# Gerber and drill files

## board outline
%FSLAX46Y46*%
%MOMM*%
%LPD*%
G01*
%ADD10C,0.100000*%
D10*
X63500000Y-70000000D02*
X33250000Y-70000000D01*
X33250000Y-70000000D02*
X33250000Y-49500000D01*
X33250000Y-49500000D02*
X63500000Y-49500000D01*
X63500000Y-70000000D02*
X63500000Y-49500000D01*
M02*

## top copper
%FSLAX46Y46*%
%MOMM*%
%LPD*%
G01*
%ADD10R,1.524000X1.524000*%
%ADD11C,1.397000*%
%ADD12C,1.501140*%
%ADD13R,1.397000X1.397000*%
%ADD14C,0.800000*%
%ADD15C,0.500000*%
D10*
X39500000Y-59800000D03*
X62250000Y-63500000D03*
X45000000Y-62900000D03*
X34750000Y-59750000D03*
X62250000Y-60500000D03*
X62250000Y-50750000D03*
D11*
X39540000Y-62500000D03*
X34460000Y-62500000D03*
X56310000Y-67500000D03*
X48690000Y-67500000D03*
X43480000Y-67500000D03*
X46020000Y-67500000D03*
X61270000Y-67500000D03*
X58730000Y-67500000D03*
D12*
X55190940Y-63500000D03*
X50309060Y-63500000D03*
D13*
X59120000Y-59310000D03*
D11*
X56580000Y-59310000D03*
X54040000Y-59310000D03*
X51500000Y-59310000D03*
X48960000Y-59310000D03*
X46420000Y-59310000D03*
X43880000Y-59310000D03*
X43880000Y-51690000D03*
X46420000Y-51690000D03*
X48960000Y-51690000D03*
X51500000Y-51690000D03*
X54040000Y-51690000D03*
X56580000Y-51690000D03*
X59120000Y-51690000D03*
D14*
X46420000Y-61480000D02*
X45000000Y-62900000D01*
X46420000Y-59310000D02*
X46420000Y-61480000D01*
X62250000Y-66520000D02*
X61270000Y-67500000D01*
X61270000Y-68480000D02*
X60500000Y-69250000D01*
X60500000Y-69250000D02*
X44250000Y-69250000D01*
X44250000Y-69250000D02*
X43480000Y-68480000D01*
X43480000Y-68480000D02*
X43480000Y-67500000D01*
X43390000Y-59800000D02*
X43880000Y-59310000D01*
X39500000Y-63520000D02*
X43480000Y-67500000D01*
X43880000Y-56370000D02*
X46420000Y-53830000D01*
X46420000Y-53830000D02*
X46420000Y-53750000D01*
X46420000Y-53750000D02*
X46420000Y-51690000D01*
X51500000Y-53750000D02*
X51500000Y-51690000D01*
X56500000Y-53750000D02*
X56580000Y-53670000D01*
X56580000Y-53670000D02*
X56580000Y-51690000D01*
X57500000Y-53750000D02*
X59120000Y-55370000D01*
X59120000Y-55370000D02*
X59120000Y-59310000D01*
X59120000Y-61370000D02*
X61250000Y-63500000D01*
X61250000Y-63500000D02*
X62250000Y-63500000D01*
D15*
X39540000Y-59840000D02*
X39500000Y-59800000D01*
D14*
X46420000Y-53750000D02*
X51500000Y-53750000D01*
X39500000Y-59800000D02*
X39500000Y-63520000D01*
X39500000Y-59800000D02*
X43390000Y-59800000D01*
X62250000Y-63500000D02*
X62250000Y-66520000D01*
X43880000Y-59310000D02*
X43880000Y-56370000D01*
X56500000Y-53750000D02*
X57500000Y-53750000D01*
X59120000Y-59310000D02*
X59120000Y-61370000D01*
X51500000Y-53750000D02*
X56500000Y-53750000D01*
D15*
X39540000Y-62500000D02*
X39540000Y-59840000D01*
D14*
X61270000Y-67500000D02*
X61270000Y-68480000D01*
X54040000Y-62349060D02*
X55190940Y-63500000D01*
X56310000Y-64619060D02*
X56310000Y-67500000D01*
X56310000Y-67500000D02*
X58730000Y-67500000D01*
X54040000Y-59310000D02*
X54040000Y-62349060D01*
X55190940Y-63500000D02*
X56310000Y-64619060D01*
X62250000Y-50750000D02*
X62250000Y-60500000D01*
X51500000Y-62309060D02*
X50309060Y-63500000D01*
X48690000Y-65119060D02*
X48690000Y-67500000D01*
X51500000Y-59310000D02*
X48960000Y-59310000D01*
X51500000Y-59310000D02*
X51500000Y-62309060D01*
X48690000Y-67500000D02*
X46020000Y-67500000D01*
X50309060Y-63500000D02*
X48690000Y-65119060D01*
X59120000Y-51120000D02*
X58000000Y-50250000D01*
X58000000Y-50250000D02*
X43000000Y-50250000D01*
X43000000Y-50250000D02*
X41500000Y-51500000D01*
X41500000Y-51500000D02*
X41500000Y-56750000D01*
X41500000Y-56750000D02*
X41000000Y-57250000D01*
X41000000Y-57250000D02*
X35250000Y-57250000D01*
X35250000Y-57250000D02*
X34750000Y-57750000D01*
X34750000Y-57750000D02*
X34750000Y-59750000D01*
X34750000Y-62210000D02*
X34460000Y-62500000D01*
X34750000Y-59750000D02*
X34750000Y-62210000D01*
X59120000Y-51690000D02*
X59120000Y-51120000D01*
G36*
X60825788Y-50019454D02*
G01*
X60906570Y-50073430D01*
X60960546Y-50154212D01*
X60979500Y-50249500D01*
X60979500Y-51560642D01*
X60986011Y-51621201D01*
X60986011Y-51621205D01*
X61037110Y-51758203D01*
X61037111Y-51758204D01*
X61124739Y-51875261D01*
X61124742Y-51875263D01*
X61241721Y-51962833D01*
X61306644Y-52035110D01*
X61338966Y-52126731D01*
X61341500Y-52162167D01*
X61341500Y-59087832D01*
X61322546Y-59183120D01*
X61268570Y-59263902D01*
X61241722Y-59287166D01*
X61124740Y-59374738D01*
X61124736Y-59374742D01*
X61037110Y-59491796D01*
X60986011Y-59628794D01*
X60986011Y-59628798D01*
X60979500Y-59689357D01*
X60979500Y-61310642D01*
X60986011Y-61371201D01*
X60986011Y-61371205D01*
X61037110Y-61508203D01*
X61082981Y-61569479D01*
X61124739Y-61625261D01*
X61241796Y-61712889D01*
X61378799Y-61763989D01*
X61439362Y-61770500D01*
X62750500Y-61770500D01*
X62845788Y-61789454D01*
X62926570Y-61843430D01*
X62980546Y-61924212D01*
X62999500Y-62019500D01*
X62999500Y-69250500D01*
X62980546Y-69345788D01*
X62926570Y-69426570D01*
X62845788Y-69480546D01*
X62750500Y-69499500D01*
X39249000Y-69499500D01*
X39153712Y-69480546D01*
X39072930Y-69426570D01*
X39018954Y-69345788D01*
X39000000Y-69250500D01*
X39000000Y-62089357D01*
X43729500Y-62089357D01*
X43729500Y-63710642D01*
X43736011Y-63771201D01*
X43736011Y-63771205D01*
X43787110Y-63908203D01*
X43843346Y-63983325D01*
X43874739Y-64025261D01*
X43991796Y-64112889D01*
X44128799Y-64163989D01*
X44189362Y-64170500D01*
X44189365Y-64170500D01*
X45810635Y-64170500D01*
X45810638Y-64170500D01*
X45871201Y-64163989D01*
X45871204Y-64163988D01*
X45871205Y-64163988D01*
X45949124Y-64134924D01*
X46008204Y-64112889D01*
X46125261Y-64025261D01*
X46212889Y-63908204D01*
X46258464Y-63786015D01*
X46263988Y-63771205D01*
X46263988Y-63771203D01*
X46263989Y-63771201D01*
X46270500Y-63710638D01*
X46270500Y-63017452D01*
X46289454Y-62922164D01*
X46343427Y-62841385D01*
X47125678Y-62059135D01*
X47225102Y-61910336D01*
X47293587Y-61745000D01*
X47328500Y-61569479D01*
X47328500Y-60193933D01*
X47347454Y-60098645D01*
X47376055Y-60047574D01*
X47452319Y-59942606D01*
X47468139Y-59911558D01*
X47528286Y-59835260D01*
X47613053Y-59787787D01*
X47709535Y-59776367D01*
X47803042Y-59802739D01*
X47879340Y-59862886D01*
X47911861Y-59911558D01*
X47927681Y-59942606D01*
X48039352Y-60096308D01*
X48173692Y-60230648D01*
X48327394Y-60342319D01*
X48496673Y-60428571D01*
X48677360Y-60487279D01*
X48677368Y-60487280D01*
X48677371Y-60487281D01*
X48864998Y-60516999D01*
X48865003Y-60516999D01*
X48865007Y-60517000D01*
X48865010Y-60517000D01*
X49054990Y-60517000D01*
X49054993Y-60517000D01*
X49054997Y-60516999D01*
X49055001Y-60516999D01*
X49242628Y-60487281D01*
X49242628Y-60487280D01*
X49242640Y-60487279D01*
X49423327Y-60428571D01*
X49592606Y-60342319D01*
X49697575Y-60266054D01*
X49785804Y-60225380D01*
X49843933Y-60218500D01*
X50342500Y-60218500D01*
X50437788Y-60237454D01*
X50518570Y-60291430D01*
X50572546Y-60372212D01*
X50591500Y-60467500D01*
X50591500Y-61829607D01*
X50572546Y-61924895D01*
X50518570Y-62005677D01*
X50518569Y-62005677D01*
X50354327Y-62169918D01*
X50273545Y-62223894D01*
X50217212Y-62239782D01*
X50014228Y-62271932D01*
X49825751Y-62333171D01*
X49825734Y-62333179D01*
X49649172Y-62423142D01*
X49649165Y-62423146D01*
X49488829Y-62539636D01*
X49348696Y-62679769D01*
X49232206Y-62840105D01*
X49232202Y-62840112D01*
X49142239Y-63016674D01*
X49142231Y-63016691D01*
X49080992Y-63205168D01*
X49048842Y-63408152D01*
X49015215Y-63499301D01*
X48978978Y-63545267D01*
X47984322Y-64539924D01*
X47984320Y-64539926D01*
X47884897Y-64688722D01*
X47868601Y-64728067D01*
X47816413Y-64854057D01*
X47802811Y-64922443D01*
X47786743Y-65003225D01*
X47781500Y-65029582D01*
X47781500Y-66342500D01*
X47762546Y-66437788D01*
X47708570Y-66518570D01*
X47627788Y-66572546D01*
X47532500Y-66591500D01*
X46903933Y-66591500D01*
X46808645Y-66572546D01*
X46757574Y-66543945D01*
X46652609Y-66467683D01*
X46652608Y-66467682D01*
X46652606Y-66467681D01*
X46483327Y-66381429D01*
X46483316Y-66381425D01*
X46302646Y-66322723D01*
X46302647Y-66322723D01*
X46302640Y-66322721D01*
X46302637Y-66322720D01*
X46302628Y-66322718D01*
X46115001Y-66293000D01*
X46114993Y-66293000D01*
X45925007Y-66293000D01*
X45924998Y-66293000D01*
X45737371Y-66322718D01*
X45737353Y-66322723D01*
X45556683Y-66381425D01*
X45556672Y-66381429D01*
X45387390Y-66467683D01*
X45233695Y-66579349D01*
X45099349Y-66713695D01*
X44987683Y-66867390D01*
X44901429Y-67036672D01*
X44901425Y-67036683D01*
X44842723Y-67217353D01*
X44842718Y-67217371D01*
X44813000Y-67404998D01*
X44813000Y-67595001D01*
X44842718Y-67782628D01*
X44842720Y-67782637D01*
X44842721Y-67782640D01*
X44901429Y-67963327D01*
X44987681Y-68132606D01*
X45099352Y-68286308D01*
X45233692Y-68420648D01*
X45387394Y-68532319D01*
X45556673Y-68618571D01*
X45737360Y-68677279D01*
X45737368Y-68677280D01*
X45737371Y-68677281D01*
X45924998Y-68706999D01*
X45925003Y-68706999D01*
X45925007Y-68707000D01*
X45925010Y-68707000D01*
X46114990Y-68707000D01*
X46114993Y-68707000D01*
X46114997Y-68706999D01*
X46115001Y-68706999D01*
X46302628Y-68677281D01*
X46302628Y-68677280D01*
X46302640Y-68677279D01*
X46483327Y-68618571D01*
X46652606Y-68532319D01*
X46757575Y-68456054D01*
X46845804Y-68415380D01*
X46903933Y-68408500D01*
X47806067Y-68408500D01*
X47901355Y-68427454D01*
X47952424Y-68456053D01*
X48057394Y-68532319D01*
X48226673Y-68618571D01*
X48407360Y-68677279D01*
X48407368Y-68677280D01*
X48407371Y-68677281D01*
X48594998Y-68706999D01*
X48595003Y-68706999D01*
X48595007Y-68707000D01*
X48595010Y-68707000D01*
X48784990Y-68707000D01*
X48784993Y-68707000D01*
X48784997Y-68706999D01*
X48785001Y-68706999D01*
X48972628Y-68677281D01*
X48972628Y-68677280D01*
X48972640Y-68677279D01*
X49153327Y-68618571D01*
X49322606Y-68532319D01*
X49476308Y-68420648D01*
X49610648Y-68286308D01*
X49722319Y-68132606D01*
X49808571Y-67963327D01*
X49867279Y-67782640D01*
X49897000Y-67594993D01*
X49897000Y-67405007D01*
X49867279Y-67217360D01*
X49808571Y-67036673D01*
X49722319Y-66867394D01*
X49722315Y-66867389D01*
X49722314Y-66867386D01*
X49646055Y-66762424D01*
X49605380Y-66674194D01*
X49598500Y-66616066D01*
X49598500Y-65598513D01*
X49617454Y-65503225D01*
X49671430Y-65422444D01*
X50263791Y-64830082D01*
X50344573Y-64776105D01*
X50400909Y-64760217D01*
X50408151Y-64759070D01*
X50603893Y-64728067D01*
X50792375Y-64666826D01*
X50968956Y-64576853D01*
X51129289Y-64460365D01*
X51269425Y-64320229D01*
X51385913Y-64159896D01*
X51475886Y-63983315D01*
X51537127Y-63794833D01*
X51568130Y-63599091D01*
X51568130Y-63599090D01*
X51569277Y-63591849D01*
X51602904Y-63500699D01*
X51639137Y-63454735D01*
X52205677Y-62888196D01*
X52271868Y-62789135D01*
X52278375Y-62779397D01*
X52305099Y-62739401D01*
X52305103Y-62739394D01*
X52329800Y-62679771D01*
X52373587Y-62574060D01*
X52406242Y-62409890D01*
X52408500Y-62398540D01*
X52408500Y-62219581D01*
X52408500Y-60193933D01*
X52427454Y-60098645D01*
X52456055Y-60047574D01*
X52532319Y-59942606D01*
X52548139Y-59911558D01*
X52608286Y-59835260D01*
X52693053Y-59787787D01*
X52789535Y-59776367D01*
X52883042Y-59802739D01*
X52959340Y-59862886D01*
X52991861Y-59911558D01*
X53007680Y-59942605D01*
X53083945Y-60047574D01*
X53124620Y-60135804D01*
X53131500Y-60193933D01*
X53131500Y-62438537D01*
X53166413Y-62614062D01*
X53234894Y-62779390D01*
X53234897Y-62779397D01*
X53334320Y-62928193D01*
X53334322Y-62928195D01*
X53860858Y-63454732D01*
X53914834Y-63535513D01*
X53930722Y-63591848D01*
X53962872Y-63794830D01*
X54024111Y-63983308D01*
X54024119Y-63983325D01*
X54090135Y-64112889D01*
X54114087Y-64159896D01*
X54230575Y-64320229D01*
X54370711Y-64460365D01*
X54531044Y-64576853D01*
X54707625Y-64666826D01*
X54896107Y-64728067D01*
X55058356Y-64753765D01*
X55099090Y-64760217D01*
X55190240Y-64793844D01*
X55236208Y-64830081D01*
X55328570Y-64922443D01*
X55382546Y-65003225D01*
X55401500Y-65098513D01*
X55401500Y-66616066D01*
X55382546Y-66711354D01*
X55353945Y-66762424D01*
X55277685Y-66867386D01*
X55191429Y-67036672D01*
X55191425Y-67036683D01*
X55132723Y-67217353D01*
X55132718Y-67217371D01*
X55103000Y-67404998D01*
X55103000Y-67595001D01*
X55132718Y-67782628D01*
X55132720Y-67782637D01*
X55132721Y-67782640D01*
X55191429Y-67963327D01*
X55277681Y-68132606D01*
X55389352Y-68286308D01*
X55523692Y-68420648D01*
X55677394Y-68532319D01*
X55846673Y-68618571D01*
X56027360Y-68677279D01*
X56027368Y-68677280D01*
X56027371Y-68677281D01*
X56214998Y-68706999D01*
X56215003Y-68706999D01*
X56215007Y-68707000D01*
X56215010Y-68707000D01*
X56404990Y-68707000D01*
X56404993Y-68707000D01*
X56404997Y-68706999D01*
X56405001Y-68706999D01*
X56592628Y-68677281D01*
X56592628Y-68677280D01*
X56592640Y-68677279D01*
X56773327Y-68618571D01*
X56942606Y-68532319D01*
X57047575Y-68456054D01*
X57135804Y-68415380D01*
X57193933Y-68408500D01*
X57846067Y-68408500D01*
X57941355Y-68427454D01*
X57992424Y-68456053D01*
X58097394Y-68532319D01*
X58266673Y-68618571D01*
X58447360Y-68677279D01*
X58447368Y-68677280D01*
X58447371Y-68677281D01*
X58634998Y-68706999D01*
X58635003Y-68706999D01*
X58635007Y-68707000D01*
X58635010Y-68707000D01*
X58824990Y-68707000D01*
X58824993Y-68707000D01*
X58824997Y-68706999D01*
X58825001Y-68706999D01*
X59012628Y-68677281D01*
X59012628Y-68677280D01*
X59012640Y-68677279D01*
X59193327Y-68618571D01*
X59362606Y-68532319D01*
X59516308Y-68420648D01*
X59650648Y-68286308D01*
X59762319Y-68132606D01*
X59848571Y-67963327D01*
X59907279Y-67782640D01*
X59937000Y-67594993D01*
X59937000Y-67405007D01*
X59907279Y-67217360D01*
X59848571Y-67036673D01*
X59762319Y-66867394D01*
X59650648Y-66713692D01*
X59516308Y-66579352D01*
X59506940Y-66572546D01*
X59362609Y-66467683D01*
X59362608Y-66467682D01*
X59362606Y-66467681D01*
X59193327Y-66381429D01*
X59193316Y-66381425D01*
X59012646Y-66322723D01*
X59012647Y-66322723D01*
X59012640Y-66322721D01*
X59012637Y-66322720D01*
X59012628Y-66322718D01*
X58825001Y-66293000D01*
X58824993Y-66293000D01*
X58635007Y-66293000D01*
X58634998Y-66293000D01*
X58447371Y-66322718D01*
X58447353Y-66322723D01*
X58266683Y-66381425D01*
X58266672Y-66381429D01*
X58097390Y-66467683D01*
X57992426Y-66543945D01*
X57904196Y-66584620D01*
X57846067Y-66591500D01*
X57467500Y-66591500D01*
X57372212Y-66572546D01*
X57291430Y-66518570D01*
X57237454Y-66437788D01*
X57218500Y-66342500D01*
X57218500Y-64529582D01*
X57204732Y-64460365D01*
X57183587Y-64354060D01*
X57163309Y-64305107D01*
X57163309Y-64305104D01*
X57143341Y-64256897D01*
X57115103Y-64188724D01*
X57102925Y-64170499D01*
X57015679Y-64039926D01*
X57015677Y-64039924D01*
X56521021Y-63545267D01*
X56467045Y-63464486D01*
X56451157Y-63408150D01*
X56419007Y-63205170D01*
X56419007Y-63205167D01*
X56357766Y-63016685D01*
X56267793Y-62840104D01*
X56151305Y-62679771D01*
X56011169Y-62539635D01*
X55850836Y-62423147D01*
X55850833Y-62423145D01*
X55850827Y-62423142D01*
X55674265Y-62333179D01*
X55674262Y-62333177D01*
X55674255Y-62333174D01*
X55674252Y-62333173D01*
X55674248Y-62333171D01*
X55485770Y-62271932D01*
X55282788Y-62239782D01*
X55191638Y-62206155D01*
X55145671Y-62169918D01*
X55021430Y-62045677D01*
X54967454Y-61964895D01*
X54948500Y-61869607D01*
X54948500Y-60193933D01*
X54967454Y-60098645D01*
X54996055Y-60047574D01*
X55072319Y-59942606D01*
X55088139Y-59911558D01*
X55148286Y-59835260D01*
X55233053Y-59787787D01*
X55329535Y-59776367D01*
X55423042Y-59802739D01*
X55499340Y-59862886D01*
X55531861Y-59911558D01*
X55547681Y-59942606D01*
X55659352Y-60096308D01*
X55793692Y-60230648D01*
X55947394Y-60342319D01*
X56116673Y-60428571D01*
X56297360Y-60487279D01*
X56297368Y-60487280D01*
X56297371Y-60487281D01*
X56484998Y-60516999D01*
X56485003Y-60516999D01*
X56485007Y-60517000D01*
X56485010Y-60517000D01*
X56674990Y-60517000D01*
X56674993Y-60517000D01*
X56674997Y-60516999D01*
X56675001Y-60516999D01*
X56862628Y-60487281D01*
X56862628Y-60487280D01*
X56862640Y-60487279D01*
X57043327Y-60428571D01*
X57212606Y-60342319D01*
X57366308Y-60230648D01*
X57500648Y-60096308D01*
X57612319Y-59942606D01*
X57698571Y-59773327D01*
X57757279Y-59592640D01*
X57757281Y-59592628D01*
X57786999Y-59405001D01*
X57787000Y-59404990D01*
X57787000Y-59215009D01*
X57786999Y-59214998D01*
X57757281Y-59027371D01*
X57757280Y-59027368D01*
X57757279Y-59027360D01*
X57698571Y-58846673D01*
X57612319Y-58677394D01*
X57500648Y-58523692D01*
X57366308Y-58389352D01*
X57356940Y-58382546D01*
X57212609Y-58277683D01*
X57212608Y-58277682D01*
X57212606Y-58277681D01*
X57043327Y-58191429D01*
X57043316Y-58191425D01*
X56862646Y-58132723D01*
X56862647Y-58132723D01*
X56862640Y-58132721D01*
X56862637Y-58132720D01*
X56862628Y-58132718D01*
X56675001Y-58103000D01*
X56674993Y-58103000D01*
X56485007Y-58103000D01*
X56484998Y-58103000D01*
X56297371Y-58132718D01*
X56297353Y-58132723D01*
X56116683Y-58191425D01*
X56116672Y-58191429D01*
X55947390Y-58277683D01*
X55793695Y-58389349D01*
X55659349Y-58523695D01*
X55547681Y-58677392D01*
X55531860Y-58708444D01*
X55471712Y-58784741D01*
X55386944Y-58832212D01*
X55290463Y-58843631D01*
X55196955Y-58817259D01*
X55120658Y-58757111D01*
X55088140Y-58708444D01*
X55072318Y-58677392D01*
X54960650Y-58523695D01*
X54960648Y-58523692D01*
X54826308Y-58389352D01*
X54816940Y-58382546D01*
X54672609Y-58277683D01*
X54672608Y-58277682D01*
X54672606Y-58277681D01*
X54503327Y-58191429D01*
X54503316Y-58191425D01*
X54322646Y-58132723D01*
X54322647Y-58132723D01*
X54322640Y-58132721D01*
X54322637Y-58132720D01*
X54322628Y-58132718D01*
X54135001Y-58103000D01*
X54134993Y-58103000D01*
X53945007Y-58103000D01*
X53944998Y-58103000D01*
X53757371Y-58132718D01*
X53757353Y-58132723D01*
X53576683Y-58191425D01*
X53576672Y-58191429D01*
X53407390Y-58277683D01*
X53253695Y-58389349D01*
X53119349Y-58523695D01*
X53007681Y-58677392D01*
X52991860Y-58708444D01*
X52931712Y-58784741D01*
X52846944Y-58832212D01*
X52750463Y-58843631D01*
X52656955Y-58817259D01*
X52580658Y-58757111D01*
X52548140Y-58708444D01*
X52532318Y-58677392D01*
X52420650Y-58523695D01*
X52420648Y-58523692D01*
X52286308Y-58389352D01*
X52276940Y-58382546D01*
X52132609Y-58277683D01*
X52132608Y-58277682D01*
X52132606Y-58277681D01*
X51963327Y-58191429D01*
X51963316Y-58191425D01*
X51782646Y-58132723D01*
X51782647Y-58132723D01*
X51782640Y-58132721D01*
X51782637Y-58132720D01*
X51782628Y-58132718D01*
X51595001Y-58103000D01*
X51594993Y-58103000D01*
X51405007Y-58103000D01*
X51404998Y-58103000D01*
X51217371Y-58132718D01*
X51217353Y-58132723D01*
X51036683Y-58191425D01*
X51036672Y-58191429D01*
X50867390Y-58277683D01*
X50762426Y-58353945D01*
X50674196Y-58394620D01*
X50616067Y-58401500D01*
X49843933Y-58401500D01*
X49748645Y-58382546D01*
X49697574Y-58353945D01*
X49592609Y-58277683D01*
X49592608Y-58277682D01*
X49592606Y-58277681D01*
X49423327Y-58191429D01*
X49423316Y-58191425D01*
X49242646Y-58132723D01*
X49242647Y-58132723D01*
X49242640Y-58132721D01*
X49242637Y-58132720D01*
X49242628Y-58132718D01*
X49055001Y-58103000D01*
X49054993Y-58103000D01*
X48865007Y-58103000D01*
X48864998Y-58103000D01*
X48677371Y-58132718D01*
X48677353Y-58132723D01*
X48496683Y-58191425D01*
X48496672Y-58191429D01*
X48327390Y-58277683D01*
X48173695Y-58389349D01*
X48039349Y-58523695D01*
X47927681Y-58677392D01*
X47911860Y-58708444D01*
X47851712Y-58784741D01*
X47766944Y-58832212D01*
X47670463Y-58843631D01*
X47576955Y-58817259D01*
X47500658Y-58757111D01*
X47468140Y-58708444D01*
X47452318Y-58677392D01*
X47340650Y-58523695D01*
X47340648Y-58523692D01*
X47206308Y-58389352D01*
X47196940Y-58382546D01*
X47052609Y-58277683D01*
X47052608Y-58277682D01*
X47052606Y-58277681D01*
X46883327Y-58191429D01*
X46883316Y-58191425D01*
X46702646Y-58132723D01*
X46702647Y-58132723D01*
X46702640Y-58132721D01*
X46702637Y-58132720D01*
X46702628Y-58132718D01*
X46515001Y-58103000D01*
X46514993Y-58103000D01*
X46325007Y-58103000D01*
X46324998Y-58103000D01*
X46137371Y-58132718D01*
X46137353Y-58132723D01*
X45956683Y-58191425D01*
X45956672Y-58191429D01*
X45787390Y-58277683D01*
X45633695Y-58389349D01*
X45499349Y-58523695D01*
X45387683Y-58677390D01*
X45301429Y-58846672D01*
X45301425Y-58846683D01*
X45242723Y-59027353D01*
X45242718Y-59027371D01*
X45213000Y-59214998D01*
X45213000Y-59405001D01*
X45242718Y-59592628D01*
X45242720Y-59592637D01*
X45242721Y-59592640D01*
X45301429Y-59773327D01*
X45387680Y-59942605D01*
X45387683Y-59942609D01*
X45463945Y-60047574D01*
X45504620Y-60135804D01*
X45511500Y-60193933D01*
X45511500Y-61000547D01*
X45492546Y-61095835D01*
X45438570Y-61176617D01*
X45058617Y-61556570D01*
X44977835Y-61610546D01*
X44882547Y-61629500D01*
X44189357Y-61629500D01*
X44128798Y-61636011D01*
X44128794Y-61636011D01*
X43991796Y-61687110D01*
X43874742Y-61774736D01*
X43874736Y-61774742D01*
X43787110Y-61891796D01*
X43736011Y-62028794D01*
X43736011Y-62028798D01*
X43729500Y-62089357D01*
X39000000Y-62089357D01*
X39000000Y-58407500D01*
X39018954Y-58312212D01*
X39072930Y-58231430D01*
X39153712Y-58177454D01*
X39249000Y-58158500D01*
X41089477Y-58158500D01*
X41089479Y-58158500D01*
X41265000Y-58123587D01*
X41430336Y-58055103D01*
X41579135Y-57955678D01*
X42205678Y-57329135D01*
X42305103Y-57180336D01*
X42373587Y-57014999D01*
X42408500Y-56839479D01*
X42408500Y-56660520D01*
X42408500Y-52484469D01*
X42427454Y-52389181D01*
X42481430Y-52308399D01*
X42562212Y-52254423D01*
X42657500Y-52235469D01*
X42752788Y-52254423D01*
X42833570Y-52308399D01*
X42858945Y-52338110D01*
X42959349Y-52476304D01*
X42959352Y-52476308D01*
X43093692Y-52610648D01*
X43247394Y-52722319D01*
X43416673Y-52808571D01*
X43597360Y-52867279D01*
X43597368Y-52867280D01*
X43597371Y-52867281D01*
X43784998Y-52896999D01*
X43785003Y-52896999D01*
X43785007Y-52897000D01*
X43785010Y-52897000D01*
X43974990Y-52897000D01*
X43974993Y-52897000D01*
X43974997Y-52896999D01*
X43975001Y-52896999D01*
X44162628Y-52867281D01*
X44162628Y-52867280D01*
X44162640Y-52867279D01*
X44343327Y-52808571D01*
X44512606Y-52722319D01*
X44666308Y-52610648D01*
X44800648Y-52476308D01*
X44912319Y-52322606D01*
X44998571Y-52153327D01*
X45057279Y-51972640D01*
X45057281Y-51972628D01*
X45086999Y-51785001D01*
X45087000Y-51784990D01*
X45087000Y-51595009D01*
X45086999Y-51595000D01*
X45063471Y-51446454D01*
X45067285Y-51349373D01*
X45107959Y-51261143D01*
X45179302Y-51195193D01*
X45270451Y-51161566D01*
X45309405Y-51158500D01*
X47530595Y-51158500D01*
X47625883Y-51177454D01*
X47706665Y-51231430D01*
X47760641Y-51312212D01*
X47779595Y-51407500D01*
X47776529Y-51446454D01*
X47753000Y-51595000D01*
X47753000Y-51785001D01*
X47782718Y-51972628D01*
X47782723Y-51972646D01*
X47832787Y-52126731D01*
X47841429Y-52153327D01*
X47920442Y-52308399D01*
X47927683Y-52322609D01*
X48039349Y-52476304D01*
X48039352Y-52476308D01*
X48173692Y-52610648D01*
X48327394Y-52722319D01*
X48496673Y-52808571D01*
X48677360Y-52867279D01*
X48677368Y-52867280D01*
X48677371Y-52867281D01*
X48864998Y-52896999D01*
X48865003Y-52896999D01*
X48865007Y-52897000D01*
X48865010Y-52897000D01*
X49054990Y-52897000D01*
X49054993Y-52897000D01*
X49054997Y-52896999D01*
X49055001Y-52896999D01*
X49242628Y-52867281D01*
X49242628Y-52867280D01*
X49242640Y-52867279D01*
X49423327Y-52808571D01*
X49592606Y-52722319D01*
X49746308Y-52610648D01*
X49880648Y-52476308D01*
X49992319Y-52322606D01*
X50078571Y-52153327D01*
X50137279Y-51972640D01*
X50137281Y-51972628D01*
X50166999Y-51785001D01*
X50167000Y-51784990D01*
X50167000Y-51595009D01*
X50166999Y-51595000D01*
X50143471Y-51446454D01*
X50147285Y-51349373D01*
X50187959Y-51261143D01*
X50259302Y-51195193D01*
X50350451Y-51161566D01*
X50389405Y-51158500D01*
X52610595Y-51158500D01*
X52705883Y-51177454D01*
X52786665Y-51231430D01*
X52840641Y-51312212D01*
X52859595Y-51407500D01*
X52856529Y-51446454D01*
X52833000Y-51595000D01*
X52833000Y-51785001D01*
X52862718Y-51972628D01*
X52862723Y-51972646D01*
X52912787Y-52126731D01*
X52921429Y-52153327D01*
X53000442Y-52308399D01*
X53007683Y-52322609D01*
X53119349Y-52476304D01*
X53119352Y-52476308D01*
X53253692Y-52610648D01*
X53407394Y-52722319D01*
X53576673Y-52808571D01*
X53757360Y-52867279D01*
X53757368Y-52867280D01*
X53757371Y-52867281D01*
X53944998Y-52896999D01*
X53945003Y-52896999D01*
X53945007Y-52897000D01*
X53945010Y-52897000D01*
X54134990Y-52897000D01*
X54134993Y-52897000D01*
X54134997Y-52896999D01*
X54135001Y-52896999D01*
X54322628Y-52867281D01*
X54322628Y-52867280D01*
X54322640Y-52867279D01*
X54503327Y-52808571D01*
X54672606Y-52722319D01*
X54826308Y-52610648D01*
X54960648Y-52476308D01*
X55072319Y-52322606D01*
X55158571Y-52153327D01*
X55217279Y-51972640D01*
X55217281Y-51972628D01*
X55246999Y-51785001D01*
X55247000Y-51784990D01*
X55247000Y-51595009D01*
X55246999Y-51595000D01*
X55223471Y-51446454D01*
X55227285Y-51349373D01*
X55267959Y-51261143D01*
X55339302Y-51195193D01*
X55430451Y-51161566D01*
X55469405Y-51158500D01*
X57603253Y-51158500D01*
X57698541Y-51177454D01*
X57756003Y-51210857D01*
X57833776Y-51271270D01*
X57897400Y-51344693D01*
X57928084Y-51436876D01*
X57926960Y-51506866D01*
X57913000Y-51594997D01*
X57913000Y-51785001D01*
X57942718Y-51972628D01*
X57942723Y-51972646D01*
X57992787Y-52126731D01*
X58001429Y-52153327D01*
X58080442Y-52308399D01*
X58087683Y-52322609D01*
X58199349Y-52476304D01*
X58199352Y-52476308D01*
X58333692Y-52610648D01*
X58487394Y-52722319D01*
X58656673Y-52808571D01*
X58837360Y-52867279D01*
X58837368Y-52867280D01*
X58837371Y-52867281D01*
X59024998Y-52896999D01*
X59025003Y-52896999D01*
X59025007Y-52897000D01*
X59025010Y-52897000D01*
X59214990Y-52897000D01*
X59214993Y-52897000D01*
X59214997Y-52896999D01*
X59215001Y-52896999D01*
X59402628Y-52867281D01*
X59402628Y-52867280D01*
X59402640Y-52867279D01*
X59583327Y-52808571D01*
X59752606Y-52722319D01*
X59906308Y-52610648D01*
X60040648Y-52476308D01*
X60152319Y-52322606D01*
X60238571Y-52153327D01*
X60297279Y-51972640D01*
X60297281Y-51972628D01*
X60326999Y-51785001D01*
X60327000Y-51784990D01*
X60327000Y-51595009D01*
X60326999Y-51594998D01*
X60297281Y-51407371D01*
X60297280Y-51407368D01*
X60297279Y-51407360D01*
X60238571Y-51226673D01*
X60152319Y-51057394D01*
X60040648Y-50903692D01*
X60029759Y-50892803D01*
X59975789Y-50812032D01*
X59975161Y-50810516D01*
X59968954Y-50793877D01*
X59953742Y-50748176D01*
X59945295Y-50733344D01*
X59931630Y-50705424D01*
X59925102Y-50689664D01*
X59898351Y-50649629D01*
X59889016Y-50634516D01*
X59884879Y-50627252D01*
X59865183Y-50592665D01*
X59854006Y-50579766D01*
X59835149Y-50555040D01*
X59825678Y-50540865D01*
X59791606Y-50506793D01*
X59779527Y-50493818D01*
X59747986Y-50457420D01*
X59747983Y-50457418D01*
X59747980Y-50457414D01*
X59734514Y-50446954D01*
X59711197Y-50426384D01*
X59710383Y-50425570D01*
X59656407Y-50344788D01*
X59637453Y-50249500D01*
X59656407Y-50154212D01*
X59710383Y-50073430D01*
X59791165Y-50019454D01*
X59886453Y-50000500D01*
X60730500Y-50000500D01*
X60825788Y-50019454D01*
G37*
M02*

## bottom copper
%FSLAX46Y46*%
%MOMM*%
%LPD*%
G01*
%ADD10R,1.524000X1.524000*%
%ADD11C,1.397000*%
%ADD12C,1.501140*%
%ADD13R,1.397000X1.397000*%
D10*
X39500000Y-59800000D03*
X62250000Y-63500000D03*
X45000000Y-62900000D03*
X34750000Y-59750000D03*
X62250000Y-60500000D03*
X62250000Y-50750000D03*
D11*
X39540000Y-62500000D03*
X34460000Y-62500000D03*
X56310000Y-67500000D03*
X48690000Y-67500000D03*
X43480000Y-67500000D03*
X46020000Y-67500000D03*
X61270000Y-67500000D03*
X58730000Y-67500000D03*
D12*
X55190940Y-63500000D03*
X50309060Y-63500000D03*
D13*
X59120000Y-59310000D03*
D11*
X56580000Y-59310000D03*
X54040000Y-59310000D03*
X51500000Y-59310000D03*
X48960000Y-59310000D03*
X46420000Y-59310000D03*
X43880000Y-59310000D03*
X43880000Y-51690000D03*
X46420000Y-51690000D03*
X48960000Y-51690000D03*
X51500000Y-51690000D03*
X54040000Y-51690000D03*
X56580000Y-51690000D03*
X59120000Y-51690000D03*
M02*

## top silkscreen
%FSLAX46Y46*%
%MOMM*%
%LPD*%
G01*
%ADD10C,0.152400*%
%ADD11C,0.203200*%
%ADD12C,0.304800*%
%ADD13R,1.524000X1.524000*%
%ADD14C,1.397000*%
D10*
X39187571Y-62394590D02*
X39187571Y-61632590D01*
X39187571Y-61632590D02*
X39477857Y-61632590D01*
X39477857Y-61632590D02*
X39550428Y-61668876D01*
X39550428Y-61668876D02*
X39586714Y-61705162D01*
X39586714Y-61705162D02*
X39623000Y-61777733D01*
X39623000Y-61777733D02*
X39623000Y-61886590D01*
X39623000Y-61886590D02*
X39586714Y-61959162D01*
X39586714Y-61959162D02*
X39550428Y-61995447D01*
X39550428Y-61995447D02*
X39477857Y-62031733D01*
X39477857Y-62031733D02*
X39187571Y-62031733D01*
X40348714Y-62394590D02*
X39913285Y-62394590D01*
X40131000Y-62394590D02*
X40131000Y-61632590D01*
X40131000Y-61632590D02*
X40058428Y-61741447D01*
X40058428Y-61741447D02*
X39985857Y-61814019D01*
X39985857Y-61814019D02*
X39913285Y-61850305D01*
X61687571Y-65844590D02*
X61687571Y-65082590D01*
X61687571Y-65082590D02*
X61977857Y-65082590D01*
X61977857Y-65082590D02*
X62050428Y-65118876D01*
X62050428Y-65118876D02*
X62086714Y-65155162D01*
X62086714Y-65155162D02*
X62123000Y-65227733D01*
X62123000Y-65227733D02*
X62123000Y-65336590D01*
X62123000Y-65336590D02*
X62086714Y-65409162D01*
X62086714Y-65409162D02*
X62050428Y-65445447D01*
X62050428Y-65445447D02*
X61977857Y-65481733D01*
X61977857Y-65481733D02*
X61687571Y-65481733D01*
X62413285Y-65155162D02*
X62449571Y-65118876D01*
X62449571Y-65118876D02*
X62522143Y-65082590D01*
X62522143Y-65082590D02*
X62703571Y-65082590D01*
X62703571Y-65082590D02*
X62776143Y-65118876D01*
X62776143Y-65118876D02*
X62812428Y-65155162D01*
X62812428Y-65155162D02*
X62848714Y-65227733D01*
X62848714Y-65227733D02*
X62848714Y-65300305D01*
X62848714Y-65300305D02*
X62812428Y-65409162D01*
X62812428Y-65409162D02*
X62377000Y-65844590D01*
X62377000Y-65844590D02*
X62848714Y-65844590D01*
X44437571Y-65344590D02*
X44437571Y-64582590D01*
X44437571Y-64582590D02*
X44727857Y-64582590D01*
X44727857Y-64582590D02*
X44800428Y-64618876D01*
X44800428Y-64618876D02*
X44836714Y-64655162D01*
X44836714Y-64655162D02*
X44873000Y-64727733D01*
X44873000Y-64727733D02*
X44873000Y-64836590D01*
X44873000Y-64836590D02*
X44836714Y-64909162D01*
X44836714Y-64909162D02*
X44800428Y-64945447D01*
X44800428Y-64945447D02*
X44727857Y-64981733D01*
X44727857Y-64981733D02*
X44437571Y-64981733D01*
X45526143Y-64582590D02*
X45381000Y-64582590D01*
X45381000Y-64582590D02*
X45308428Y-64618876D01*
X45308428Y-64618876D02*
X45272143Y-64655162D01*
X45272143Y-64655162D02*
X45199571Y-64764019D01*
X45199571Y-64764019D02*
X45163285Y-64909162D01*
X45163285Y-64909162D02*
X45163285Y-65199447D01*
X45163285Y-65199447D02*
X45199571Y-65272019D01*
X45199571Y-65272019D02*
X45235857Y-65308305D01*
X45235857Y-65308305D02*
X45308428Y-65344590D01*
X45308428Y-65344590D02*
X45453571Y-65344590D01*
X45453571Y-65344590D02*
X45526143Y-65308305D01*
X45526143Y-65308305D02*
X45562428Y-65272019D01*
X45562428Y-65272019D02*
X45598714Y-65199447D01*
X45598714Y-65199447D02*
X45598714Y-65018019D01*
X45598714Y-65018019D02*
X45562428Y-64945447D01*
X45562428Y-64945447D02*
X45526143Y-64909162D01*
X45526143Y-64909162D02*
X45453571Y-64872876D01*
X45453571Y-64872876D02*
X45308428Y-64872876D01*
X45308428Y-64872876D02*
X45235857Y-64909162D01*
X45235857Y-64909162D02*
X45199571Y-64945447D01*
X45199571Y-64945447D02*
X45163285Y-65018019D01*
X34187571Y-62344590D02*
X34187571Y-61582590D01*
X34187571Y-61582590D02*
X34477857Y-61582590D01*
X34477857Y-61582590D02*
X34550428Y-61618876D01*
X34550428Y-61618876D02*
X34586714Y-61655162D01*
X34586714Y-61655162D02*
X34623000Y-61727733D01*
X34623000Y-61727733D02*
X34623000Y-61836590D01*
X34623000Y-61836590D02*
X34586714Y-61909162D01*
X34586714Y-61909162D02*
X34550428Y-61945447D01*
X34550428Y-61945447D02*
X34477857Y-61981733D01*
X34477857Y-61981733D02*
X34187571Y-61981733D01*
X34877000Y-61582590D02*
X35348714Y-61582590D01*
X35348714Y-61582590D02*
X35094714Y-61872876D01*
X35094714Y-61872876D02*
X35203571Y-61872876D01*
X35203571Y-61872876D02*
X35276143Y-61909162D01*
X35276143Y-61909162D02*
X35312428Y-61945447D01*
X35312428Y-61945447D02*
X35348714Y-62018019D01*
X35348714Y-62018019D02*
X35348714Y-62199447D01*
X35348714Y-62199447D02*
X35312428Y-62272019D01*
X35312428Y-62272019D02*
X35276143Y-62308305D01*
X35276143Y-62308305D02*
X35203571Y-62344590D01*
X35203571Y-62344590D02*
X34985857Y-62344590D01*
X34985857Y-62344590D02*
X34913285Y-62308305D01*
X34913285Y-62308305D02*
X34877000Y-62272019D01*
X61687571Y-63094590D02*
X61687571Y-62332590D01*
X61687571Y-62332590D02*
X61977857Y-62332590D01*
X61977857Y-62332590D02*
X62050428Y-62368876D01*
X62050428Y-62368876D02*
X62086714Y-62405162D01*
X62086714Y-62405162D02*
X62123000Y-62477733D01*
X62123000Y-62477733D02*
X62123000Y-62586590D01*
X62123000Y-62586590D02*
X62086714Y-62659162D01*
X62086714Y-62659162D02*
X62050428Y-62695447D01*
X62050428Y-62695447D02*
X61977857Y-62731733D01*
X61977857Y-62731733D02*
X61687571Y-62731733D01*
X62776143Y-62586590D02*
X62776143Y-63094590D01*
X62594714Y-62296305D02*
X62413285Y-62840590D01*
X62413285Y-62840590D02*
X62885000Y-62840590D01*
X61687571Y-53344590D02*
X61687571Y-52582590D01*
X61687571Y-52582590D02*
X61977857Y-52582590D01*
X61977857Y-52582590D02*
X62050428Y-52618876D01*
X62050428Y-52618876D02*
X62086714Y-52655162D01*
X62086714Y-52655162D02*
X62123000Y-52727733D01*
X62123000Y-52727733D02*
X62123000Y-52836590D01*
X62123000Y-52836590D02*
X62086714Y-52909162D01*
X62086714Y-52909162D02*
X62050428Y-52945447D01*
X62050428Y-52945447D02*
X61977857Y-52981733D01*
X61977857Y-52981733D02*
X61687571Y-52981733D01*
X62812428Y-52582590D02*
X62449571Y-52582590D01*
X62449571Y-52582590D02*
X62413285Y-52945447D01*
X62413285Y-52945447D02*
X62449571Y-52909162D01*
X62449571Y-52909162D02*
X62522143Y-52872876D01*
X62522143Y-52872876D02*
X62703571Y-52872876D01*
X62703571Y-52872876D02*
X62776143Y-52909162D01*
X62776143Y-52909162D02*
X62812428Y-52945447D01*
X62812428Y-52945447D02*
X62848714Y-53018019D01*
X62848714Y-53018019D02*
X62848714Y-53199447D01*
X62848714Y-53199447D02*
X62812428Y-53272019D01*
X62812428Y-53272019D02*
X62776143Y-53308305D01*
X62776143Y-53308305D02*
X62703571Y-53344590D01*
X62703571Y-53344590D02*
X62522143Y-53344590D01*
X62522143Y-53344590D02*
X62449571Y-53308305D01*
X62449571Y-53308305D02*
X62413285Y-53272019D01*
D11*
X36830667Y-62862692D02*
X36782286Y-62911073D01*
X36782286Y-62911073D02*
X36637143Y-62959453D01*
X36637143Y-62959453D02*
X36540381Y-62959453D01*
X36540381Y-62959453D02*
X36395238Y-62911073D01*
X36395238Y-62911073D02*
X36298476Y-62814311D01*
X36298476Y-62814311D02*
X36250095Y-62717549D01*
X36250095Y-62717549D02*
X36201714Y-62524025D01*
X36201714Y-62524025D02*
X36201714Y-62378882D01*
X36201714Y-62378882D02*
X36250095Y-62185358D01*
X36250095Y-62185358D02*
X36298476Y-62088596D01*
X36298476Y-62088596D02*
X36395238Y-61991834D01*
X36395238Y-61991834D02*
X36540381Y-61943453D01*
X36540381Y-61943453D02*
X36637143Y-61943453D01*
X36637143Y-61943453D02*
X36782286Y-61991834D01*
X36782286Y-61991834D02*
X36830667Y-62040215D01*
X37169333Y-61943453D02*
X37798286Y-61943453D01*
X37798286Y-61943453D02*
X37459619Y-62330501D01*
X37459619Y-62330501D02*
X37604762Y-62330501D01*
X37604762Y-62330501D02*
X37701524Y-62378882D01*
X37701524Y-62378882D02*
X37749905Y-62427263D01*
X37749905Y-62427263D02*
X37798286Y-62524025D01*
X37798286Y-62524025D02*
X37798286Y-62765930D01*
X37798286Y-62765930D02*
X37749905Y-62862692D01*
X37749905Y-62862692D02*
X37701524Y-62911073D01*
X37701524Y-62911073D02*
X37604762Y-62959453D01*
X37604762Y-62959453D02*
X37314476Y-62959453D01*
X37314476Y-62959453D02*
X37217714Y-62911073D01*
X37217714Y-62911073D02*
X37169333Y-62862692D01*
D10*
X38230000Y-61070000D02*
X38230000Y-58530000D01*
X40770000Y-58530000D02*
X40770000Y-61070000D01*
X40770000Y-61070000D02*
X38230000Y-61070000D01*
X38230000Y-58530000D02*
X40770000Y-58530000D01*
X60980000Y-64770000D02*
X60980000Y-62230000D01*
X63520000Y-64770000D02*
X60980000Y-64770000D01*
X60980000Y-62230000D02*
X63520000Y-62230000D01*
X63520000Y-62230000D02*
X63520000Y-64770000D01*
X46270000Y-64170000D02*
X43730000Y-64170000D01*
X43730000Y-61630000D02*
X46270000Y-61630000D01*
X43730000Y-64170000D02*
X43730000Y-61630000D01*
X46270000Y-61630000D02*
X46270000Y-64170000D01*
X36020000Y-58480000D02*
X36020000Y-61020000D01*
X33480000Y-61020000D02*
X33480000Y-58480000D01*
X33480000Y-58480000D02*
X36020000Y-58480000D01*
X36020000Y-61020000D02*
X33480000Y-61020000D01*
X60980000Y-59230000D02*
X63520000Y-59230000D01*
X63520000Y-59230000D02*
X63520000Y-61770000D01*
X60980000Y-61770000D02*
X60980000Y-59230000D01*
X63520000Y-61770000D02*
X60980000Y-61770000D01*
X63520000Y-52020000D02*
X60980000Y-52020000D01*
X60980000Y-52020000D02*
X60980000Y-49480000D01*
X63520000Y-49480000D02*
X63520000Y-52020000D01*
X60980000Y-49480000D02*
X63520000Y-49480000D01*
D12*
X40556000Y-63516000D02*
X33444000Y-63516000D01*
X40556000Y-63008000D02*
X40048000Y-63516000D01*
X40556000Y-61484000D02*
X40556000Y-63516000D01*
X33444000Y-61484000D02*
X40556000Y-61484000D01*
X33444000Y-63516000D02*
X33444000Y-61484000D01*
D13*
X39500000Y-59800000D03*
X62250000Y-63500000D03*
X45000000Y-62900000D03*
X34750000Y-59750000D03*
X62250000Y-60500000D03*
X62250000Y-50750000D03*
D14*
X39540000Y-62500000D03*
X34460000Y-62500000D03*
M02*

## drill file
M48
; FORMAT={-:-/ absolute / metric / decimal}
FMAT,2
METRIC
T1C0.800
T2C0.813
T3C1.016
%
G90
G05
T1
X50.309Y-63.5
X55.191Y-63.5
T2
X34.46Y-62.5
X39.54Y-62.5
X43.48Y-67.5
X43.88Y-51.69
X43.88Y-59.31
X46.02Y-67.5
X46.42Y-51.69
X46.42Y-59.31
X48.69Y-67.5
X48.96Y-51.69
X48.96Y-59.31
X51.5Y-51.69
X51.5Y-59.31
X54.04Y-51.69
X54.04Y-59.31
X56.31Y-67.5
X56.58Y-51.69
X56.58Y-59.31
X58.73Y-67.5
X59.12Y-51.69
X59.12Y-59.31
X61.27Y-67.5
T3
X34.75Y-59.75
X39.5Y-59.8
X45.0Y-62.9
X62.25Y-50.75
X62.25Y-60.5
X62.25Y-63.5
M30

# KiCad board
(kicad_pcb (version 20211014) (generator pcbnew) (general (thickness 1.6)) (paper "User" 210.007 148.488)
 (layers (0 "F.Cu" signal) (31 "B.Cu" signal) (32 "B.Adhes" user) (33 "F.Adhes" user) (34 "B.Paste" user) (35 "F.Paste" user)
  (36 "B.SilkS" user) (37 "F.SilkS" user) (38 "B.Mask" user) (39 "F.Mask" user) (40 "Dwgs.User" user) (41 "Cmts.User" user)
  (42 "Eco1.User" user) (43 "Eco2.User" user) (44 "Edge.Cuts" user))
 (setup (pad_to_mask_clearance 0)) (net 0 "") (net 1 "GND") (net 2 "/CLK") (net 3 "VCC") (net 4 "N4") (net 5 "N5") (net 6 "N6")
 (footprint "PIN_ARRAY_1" (layer "F.Cu") (at 39.5 59.8)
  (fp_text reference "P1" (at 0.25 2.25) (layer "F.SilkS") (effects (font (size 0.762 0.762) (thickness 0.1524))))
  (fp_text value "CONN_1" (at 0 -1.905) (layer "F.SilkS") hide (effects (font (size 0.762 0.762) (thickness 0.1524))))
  (fp_line (start -1.27 1.27) (end -1.27 -1.27) (layer "F.SilkS") (width 0.1524))
  (fp_line (start 1.27 -1.27) (end 1.27 1.27) (layer "F.SilkS") (width 0.1524))
  (fp_line (start 1.27 1.27) (end -1.27 1.27) (layer "F.SilkS") (width 0.1524))
  (fp_line (start -1.27 -1.27) (end 1.27 -1.27) (layer "F.SilkS") (width 0.1524))
  (pad "1" thru_hole rect locked (at 0 0) (size 1.524 1.524) (drill 1.016) (layers *.Cu *.Mask "F.SilkS") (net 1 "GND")))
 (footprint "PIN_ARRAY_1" (layer "F.Cu") (at 62.25 63.5)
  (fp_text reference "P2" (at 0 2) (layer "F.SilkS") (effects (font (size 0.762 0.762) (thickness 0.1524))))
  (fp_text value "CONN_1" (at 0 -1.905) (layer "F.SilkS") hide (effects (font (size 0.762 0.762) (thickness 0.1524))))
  (fp_line (start -1.27 1.27) (end -1.27 -1.27) (layer "F.SilkS") (width 0.1524))
  (fp_line (start 1.27 1.27) (end -1.27 1.27) (layer "F.SilkS") (width 0.1524))
  (fp_line (start -1.27 -1.27) (end 1.27 -1.27) (layer "F.SilkS") (width 0.1524))
  (fp_line (start 1.27 -1.27) (end 1.27 1.27) (layer "F.SilkS") (width 0.1524))
  (pad "1" thru_hole rect locked (at 0 0) (size 1.524 1.524) (drill 1.016) (layers *.Cu *.Mask "F.SilkS") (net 1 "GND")))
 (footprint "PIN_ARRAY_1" (layer "F.Cu") (at 45 62.9)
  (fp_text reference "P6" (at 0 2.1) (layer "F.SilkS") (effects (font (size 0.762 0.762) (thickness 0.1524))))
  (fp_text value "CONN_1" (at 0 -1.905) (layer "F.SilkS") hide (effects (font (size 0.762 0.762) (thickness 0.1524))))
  (fp_line (start 1.27 1.27) (end -1.27 1.27) (layer "F.SilkS") (width 0.1524))
  (fp_line (start -1.27 -1.27) (end 1.27 -1.27) (layer "F.SilkS") (width 0.1524))
  (fp_line (start -1.27 1.27) (end -1.27 -1.27) (layer "F.SilkS") (width 0.1524))
  (fp_line (start 1.27 -1.27) (end 1.27 1.27) (layer "F.SilkS") (width 0.1524))
  (pad "1" thru_hole rect locked (at 0 0) (size 1.524 1.524) (drill 1.016) (layers *.Cu *.Mask "F.SilkS") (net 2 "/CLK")))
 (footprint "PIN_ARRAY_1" (layer "F.Cu") (at 34.75 59.75)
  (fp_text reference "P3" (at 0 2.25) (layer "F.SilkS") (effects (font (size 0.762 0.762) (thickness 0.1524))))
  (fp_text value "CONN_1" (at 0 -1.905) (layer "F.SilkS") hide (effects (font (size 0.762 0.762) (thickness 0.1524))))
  (fp_line (start 1.27 -1.27) (end 1.27 1.27) (layer "F.SilkS") (width 0.1524))
  (fp_line (start -1.27 1.27) (end -1.27 -1.27) (layer "F.SilkS") (width 0.1524))
  (fp_line (start -1.27 -1.27) (end 1.27 -1.27) (layer "F.SilkS") (width 0.1524))
  (fp_line (start 1.27 1.27) (end -1.27 1.27) (layer "F.SilkS") (width 0.1524))
  (pad "1" thru_hole rect locked (at 0 0) (size 1.524 1.524) (drill 1.016) (layers *.Cu *.Mask "F.SilkS") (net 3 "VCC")))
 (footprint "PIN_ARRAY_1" (layer "F.Cu") (at 62.25 60.5)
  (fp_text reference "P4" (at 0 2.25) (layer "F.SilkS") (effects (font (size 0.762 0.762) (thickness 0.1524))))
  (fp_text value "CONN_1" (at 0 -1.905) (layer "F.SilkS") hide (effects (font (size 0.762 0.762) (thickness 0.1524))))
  (fp_line (start -1.27 -1.27) (end 1.27 -1.27) (layer "F.SilkS") (width 0.1524))
  (fp_line (start 1.27 -1.27) (end 1.27 1.27) (layer "F.SilkS") (width 0.1524))
  (fp_line (start -1.27 1.27) (end -1.27 -1.27) (layer "F.SilkS") (width 0.1524))
  (fp_line (start 1.27 1.27) (end -1.27 1.27) (layer "F.SilkS") (width 0.1524))
  (pad "1" thru_hole rect locked (at 0 0) (size 1.524 1.524) (drill 1.016) (layers *.Cu *.Mask "F.SilkS") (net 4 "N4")))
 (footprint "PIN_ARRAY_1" (layer "F.Cu") (at 62.25 50.75)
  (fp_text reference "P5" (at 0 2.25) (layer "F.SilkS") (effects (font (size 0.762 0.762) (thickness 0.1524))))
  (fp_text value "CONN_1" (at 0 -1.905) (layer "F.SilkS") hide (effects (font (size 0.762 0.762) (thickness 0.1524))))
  (fp_line (start 1.27 1.27) (end -1.27 1.27) (layer "F.SilkS") (width 0.1524))
  (fp_line (start -1.27 1.27) (end -1.27 -1.27) (layer "F.SilkS") (width 0.1524))
  (fp_line (start 1.27 -1.27) (end 1.27 1.27) (layer "F.SilkS") (width 0.1524))
  (fp_line (start -1.27 -1.27) (end 1.27 -1.27) (layer "F.SilkS") (width 0.1524))
  (pad "1" thru_hole rect locked (at 0 0) (size 1.524 1.524) (drill 1.016) (layers *.Cu *.Mask "F.SilkS") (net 4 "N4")))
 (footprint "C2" (layer "F.Cu") (at 37 62.5 180)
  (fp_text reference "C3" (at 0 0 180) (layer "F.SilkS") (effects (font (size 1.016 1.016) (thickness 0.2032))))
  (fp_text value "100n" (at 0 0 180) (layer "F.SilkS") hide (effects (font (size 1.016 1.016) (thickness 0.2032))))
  (fp_line (start -3.556 -1.016) (end 3.556 -1.016) (layer "F.SilkS") (width 0.3048))
  (fp_line (start -3.556 -0.508) (end -3.048 -1.016) (layer "F.SilkS") (width 0.3048))
  (fp_line (start -3.556 1.016) (end -3.556 -1.016) (layer "F.SilkS") (width 0.3048))
  (fp_line (start 3.556 1.016) (end -3.556 1.016) (layer "F.SilkS") (width 0.3048))
  (fp_line (start 3.556 -1.016) (end 3.556 1.016) (layer "F.SilkS") (width 0.3048))
  (pad "1" thru_hole circle locked (at -2.54 0 180) (size 1.397 1.397) (drill 0.8128) (layers *.Cu *.Mask "F.SilkS") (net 1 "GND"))
  (pad "2" thru_hole circle locked (at 2.54 0 180) (size 1.397 1.397) (drill 0.8128) (layers *.Cu *.Mask "F.SilkS") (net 3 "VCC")))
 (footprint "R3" (layer "B.Cu") (at 52.5 67.5 180) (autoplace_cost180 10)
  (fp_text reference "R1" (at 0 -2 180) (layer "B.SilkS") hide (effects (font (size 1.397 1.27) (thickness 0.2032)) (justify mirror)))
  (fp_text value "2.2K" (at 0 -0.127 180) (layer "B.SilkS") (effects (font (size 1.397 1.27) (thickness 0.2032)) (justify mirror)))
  (pad "1" thru_hole circle locked (at -3.81 0 180) (size 1.397 1.397) (drill 0.8128) (layers *.Cu *.Mask "B.SilkS") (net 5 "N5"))
  (pad "2" thru_hole circle locked (at 3.81 0 180) (size 1.397 1.397) (drill 0.8128) (layers *.Cu *.Mask "B.SilkS") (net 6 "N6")))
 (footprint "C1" (layer "B.Cu") (at 44.75 67.5)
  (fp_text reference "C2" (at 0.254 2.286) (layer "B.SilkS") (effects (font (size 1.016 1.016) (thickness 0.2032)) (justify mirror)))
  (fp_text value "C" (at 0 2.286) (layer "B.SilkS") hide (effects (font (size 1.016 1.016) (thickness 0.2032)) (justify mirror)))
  (pad "1" thru_hole circle locked (at -1.27 0) (size 1.397 1.397) (drill 0.8128) (layers *.Cu *.Mask "B.SilkS") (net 1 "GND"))
  (pad "2" thru_hole circle locked (at 1.27 0) (size 1.397 1.397) (drill 0.8128) (layers *.Cu *.Mask "B.SilkS") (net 6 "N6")))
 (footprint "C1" (layer "B.Cu") (at 60 67.5 180)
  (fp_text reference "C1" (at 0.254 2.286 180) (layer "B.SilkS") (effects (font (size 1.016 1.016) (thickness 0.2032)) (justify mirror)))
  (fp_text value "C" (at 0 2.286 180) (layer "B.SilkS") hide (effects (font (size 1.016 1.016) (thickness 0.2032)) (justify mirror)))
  (pad "1" thru_hole circle locked (at -1.27 0 180) (size 1.397 1.397) (drill 0.8128) (layers *.Cu *.Mask "B.SilkS") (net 1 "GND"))
  (pad "2" thru_hole circle locked (at 1.27 0 180) (size 1.397 1.397) (drill 0.8128) (layers *.Cu *.Mask "B.SilkS") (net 5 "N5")))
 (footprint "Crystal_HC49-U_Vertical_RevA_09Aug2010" (layer "B.Cu") (at 52.75 63.5 180)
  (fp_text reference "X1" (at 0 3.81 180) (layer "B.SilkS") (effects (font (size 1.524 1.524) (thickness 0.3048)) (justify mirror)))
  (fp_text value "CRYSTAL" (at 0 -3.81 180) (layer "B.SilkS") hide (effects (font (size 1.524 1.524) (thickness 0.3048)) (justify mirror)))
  (pad "1" thru_hole circle locked (at -2.44094 0 180) (size 1.50114 1.50114) (drill 0.8001) (layers *.Cu *.Mask "B.SilkS") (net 5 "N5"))
  (pad "2" thru_hole circle locked (at 2.44094 0 180) (size 1.50114 1.50114) (drill 0.8001) (layers *.Cu *.Mask "B.SilkS") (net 6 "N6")))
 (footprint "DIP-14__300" (layer "B.Cu") (at 51.5 55.5 180)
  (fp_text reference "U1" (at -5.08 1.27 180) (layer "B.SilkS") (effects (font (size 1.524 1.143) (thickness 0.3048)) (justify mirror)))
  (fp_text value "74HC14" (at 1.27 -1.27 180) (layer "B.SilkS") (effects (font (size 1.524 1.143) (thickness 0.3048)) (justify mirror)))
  (pad "1" thru_hole rect locked (at -7.62 -3.81 180) (size 1.397 1.397) (drill 0.8128) (layers *.Cu *.Mask "B.SilkS") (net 1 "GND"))
  (pad "2" thru_hole circle locked (at -5.08 -3.81 180) (size 1.397 1.397) (drill 0.8128) (layers *.Cu *.Mask "B.SilkS"))
  (pad "3" thru_hole circle locked (at -2.54 -3.81 180) (size 1.397 1.397) (drill 0.8128) (layers *.Cu *.Mask "B.SilkS") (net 5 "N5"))
  (pad "4" thru_hole circle locked (at 0 -3.81 180) (size 1.397 1.397) (drill 0.8128) (layers *.Cu *.Mask "B.SilkS") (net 6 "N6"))
  (pad "5" thru_hole circle locked (at 2.54 -3.81 180) (size 1.397 1.397) (drill 0.8128) (layers *.Cu *.Mask "B.SilkS") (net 6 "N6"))
  (pad "6" thru_hole circle locked (at 5.08 -3.81 180) (size 1.397 1.397) (drill 0.8128) (layers *.Cu *.Mask "B.SilkS") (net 2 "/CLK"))
  (pad "7" thru_hole circle locked (at 7.62 -3.81 180) (size 1.397 1.397) (drill 0.8128) (layers *.Cu *.Mask "B.SilkS") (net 1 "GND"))
  (pad "8" thru_hole circle locked (at 7.62 3.81 180) (size 1.397 1.397) (drill 0.8128) (layers *.Cu *.Mask "B.SilkS"))
  (pad "9" thru_hole circle locked (at 5.08 3.81 180) (size 1.397 1.397) (drill 0.8128) (layers *.Cu *.Mask "B.SilkS") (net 1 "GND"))
  (pad "10" thru_hole circle locked (at 2.54 3.81 180) (size 1.397 1.397) (drill 0.8128) (layers *.Cu *.Mask "B.SilkS"))
  (pad "11" thru_hole circle locked (at 0 3.81 180) (size 1.397 1.397) (drill 0.8128) (layers *.Cu *.Mask "B.SilkS") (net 1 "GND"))
  (pad "12" thru_hole circle locked (at -2.54 3.81 180) (size 1.397 1.397) (drill 0.8128) (layers *.Cu *.Mask "B.SilkS"))
  (pad "13" thru_hole circle locked (at -5.08 3.81 180) (size 1.397 1.397) (drill 0.8128) (layers *.Cu *.Mask "B.SilkS") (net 1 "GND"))
  (pad "14" thru_hole circle locked (at -7.62 3.81 180) (size 1.397 1.397) (drill 0.8128) (layers *.Cu *.Mask "B.SilkS") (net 3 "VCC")))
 (gr_line (start 63.5 70) (end 33.25 70) (layer "Edge.Cuts") (width 0.1))
 (gr_line (start 33.25 70) (end 33.25 49.5) (layer "Edge.Cuts") (width 0.1))
 (gr_line (start 33.25 49.5) (end 63.5 49.5) (layer "Edge.Cuts") (width 0.1))
 (gr_line (start 63.5 70) (end 63.5 49.5) (layer "Edge.Cuts") (width 0.1))
 (segment (start 46.42 61.48) (end 45 62.9) (width 0.8) (layer "F.Cu") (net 2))
 (segment (start 46.42 59.31) (end 46.42 61.48) (width 0.8) (layer "F.Cu") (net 2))
 (segment (start 62.25 66.52) (end 61.27 67.5) (width 0.8) (layer "F.Cu") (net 1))
 (segment (start 61.27 68.48) (end 60.5 69.25) (width 0.8) (layer "F.Cu") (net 1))
 (segment (start 60.5 69.25) (end 44.25 69.25) (width 0.8) (layer "F.Cu") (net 1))
 (segment (start 44.25 69.25) (end 43.48 68.48) (width 0.8) (layer "F.Cu") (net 1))
 (segment (start 43.48 68.48) (end 43.48 67.5) (width 0.8) (layer "F.Cu") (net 1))
 (segment (start 43.39 59.8) (end 43.88 59.31) (width 0.8) (layer "F.Cu") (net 1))
 (segment (start 39.5 63.52) (end 43.48 67.5) (width 0.8) (layer "F.Cu") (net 1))
 (segment (start 43.88 56.37) (end 46.42 53.83) (width 0.8) (layer "F.Cu") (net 1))
 (segment (start 46.42 53.83) (end 46.42 53.75) (width 0.8) (layer "F.Cu") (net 1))
 (segment (start 46.42 53.75) (end 46.42 51.69) (width 0.8) (layer "F.Cu") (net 1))
 (segment (start 51.5 53.75) (end 51.5 51.69) (width 0.8) (layer "F.Cu") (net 1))
 (segment (start 56.5 53.75) (end 56.58 53.67) (width 0.8) (layer "F.Cu") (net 1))
 (segment (start 56.58 53.67) (end 56.58 51.69) (width 0.8) (layer "F.Cu") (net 1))
 (segment (start 57.5 53.75) (end 59.12 55.37) (width 0.8) (layer "F.Cu") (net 1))
 (segment (start 59.12 55.37) (end 59.12 59.31) (width 0.8) (layer "F.Cu") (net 1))
 (segment (start 59.12 61.37) (end 61.25 63.5) (width 0.8) (layer "F.Cu") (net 1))
 (segment (start 61.25 63.5) (end 62.25 63.5) (width 0.8) (layer "F.Cu") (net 1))
 (segment (start 39.54 59.84) (end 39.5 59.8) (width 0.5) (layer "F.Cu") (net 1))
 (segment (start 46.42 53.75) (end 51.5 53.75) (width 0.8) (layer "F.Cu") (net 1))
 (segment (start 39.5 59.8) (end 39.5 63.52) (width 0.8) (layer "F.Cu") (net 1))
 (segment (start 39.5 59.8) (end 43.39 59.8) (width 0.8) (layer "F.Cu") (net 1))
 (segment (start 62.25 63.5) (end 62.25 66.52) (width 0.8) (layer "F.Cu") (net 1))
 (segment (start 43.88 59.31) (end 43.88 56.37) (width 0.8) (layer "F.Cu") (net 1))
 (segment (start 56.5 53.75) (end 57.5 53.75) (width 0.8) (layer "F.Cu") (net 1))
 (segment (start 59.12 59.31) (end 59.12 61.37) (width 0.8) (layer "F.Cu") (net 1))
 (segment (start 51.5 53.75) (end 56.5 53.75) (width 0.8) (layer "F.Cu") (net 1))
 (segment (start 39.54 62.5) (end 39.54 59.84) (width 0.5) (layer "F.Cu") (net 1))
 (segment (start 61.27 67.5) (end 61.27 68.48) (width 0.8) (layer "F.Cu") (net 1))
 (segment (start 54.04 62.34906) (end 55.19094 63.5) (width 0.8) (layer "F.Cu") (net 5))
 (segment (start 56.31 64.61906) (end 56.31 67.5) (width 0.8) (layer "F.Cu") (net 5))
 (segment (start 56.31 67.5) (end 58.73 67.5) (width 0.8) (layer "F.Cu") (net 5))
 (segment (start 54.04 59.31) (end 54.04 62.34906) (width 0.8) (layer "F.Cu") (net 5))
 (segment (start 55.19094 63.5) (end 56.31 64.61906) (width 0.8) (layer "F.Cu") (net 5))
 (segment (start 62.25 50.75) (end 62.25 60.5) (width 0.8) (layer "F.Cu") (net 4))
 (segment (start 51.5 62.30906) (end 50.30906 63.5) (width 0.8) (layer "F.Cu") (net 6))
 (segment (start 48.69 65.11906) (end 48.69 67.5) (width 0.8) (layer "F.Cu") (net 6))
 (segment (start 51.5 59.31) (end 48.96 59.31) (width 0.8) (layer "F.Cu") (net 6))
 (segment (start 51.5 59.31) (end 51.5 62.30906) (width 0.8) (layer "F.Cu") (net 6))
 (segment (start 48.69 67.5) (end 46.02 67.5) (width 0.8) (layer "F.Cu") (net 6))
 (segment (start 50.30906 63.5) (end 48.69 65.11906) (width 0.8) (layer "F.Cu") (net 6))
 (segment (start 59.12 51.12) (end 58 50.25) (width 0.8) (layer "F.Cu") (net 3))
 (segment (start 58 50.25) (end 43 50.25) (width 0.8) (layer "F.Cu") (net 3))
 (segment (start 43 50.25) (end 41.5 51.5) (width 0.8) (layer "F.Cu") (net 3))
 (segment (start 41.5 51.5) (end 41.5 56.75) (width 0.8) (layer "F.Cu") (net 3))
 (segment (start 41.5 56.75) (end 41 57.25) (width 0.8) (layer "F.Cu") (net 3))
 (segment (start 41 57.25) (end 35.25 57.25) (width 0.8) (layer "F.Cu") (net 3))
 (segment (start 35.25 57.25) (end 34.75 57.75) (width 0.8) (layer "F.Cu") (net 3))
 (segment (start 34.75 57.75) (end 34.75 59.75) (width 0.8) (layer "F.Cu") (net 3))
 (segment (start 34.75 62.21) (end 34.46 62.5) (width 0.8) (layer "F.Cu") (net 3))
 (segment (start 34.75 59.75) (end 34.75 62.21) (width 0.8) (layer "F.Cu") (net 3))
 (segment (start 59.12 51.69) (end 59.12 51.12) (width 0.8) (layer "F.Cu") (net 3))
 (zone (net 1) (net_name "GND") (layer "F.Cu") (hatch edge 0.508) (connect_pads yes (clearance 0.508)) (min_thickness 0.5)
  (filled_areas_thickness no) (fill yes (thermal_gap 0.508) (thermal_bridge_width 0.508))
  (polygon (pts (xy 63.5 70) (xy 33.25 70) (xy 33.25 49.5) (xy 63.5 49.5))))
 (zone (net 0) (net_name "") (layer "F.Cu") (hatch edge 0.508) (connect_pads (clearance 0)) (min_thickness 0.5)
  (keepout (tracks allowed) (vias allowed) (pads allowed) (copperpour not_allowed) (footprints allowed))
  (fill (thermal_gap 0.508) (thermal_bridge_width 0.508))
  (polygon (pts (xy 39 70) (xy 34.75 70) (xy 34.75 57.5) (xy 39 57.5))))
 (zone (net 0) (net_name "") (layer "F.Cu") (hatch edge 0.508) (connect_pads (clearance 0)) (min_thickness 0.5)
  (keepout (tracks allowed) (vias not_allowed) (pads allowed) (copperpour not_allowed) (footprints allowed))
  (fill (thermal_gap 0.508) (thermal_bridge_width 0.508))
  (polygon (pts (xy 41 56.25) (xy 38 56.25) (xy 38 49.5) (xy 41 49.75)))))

